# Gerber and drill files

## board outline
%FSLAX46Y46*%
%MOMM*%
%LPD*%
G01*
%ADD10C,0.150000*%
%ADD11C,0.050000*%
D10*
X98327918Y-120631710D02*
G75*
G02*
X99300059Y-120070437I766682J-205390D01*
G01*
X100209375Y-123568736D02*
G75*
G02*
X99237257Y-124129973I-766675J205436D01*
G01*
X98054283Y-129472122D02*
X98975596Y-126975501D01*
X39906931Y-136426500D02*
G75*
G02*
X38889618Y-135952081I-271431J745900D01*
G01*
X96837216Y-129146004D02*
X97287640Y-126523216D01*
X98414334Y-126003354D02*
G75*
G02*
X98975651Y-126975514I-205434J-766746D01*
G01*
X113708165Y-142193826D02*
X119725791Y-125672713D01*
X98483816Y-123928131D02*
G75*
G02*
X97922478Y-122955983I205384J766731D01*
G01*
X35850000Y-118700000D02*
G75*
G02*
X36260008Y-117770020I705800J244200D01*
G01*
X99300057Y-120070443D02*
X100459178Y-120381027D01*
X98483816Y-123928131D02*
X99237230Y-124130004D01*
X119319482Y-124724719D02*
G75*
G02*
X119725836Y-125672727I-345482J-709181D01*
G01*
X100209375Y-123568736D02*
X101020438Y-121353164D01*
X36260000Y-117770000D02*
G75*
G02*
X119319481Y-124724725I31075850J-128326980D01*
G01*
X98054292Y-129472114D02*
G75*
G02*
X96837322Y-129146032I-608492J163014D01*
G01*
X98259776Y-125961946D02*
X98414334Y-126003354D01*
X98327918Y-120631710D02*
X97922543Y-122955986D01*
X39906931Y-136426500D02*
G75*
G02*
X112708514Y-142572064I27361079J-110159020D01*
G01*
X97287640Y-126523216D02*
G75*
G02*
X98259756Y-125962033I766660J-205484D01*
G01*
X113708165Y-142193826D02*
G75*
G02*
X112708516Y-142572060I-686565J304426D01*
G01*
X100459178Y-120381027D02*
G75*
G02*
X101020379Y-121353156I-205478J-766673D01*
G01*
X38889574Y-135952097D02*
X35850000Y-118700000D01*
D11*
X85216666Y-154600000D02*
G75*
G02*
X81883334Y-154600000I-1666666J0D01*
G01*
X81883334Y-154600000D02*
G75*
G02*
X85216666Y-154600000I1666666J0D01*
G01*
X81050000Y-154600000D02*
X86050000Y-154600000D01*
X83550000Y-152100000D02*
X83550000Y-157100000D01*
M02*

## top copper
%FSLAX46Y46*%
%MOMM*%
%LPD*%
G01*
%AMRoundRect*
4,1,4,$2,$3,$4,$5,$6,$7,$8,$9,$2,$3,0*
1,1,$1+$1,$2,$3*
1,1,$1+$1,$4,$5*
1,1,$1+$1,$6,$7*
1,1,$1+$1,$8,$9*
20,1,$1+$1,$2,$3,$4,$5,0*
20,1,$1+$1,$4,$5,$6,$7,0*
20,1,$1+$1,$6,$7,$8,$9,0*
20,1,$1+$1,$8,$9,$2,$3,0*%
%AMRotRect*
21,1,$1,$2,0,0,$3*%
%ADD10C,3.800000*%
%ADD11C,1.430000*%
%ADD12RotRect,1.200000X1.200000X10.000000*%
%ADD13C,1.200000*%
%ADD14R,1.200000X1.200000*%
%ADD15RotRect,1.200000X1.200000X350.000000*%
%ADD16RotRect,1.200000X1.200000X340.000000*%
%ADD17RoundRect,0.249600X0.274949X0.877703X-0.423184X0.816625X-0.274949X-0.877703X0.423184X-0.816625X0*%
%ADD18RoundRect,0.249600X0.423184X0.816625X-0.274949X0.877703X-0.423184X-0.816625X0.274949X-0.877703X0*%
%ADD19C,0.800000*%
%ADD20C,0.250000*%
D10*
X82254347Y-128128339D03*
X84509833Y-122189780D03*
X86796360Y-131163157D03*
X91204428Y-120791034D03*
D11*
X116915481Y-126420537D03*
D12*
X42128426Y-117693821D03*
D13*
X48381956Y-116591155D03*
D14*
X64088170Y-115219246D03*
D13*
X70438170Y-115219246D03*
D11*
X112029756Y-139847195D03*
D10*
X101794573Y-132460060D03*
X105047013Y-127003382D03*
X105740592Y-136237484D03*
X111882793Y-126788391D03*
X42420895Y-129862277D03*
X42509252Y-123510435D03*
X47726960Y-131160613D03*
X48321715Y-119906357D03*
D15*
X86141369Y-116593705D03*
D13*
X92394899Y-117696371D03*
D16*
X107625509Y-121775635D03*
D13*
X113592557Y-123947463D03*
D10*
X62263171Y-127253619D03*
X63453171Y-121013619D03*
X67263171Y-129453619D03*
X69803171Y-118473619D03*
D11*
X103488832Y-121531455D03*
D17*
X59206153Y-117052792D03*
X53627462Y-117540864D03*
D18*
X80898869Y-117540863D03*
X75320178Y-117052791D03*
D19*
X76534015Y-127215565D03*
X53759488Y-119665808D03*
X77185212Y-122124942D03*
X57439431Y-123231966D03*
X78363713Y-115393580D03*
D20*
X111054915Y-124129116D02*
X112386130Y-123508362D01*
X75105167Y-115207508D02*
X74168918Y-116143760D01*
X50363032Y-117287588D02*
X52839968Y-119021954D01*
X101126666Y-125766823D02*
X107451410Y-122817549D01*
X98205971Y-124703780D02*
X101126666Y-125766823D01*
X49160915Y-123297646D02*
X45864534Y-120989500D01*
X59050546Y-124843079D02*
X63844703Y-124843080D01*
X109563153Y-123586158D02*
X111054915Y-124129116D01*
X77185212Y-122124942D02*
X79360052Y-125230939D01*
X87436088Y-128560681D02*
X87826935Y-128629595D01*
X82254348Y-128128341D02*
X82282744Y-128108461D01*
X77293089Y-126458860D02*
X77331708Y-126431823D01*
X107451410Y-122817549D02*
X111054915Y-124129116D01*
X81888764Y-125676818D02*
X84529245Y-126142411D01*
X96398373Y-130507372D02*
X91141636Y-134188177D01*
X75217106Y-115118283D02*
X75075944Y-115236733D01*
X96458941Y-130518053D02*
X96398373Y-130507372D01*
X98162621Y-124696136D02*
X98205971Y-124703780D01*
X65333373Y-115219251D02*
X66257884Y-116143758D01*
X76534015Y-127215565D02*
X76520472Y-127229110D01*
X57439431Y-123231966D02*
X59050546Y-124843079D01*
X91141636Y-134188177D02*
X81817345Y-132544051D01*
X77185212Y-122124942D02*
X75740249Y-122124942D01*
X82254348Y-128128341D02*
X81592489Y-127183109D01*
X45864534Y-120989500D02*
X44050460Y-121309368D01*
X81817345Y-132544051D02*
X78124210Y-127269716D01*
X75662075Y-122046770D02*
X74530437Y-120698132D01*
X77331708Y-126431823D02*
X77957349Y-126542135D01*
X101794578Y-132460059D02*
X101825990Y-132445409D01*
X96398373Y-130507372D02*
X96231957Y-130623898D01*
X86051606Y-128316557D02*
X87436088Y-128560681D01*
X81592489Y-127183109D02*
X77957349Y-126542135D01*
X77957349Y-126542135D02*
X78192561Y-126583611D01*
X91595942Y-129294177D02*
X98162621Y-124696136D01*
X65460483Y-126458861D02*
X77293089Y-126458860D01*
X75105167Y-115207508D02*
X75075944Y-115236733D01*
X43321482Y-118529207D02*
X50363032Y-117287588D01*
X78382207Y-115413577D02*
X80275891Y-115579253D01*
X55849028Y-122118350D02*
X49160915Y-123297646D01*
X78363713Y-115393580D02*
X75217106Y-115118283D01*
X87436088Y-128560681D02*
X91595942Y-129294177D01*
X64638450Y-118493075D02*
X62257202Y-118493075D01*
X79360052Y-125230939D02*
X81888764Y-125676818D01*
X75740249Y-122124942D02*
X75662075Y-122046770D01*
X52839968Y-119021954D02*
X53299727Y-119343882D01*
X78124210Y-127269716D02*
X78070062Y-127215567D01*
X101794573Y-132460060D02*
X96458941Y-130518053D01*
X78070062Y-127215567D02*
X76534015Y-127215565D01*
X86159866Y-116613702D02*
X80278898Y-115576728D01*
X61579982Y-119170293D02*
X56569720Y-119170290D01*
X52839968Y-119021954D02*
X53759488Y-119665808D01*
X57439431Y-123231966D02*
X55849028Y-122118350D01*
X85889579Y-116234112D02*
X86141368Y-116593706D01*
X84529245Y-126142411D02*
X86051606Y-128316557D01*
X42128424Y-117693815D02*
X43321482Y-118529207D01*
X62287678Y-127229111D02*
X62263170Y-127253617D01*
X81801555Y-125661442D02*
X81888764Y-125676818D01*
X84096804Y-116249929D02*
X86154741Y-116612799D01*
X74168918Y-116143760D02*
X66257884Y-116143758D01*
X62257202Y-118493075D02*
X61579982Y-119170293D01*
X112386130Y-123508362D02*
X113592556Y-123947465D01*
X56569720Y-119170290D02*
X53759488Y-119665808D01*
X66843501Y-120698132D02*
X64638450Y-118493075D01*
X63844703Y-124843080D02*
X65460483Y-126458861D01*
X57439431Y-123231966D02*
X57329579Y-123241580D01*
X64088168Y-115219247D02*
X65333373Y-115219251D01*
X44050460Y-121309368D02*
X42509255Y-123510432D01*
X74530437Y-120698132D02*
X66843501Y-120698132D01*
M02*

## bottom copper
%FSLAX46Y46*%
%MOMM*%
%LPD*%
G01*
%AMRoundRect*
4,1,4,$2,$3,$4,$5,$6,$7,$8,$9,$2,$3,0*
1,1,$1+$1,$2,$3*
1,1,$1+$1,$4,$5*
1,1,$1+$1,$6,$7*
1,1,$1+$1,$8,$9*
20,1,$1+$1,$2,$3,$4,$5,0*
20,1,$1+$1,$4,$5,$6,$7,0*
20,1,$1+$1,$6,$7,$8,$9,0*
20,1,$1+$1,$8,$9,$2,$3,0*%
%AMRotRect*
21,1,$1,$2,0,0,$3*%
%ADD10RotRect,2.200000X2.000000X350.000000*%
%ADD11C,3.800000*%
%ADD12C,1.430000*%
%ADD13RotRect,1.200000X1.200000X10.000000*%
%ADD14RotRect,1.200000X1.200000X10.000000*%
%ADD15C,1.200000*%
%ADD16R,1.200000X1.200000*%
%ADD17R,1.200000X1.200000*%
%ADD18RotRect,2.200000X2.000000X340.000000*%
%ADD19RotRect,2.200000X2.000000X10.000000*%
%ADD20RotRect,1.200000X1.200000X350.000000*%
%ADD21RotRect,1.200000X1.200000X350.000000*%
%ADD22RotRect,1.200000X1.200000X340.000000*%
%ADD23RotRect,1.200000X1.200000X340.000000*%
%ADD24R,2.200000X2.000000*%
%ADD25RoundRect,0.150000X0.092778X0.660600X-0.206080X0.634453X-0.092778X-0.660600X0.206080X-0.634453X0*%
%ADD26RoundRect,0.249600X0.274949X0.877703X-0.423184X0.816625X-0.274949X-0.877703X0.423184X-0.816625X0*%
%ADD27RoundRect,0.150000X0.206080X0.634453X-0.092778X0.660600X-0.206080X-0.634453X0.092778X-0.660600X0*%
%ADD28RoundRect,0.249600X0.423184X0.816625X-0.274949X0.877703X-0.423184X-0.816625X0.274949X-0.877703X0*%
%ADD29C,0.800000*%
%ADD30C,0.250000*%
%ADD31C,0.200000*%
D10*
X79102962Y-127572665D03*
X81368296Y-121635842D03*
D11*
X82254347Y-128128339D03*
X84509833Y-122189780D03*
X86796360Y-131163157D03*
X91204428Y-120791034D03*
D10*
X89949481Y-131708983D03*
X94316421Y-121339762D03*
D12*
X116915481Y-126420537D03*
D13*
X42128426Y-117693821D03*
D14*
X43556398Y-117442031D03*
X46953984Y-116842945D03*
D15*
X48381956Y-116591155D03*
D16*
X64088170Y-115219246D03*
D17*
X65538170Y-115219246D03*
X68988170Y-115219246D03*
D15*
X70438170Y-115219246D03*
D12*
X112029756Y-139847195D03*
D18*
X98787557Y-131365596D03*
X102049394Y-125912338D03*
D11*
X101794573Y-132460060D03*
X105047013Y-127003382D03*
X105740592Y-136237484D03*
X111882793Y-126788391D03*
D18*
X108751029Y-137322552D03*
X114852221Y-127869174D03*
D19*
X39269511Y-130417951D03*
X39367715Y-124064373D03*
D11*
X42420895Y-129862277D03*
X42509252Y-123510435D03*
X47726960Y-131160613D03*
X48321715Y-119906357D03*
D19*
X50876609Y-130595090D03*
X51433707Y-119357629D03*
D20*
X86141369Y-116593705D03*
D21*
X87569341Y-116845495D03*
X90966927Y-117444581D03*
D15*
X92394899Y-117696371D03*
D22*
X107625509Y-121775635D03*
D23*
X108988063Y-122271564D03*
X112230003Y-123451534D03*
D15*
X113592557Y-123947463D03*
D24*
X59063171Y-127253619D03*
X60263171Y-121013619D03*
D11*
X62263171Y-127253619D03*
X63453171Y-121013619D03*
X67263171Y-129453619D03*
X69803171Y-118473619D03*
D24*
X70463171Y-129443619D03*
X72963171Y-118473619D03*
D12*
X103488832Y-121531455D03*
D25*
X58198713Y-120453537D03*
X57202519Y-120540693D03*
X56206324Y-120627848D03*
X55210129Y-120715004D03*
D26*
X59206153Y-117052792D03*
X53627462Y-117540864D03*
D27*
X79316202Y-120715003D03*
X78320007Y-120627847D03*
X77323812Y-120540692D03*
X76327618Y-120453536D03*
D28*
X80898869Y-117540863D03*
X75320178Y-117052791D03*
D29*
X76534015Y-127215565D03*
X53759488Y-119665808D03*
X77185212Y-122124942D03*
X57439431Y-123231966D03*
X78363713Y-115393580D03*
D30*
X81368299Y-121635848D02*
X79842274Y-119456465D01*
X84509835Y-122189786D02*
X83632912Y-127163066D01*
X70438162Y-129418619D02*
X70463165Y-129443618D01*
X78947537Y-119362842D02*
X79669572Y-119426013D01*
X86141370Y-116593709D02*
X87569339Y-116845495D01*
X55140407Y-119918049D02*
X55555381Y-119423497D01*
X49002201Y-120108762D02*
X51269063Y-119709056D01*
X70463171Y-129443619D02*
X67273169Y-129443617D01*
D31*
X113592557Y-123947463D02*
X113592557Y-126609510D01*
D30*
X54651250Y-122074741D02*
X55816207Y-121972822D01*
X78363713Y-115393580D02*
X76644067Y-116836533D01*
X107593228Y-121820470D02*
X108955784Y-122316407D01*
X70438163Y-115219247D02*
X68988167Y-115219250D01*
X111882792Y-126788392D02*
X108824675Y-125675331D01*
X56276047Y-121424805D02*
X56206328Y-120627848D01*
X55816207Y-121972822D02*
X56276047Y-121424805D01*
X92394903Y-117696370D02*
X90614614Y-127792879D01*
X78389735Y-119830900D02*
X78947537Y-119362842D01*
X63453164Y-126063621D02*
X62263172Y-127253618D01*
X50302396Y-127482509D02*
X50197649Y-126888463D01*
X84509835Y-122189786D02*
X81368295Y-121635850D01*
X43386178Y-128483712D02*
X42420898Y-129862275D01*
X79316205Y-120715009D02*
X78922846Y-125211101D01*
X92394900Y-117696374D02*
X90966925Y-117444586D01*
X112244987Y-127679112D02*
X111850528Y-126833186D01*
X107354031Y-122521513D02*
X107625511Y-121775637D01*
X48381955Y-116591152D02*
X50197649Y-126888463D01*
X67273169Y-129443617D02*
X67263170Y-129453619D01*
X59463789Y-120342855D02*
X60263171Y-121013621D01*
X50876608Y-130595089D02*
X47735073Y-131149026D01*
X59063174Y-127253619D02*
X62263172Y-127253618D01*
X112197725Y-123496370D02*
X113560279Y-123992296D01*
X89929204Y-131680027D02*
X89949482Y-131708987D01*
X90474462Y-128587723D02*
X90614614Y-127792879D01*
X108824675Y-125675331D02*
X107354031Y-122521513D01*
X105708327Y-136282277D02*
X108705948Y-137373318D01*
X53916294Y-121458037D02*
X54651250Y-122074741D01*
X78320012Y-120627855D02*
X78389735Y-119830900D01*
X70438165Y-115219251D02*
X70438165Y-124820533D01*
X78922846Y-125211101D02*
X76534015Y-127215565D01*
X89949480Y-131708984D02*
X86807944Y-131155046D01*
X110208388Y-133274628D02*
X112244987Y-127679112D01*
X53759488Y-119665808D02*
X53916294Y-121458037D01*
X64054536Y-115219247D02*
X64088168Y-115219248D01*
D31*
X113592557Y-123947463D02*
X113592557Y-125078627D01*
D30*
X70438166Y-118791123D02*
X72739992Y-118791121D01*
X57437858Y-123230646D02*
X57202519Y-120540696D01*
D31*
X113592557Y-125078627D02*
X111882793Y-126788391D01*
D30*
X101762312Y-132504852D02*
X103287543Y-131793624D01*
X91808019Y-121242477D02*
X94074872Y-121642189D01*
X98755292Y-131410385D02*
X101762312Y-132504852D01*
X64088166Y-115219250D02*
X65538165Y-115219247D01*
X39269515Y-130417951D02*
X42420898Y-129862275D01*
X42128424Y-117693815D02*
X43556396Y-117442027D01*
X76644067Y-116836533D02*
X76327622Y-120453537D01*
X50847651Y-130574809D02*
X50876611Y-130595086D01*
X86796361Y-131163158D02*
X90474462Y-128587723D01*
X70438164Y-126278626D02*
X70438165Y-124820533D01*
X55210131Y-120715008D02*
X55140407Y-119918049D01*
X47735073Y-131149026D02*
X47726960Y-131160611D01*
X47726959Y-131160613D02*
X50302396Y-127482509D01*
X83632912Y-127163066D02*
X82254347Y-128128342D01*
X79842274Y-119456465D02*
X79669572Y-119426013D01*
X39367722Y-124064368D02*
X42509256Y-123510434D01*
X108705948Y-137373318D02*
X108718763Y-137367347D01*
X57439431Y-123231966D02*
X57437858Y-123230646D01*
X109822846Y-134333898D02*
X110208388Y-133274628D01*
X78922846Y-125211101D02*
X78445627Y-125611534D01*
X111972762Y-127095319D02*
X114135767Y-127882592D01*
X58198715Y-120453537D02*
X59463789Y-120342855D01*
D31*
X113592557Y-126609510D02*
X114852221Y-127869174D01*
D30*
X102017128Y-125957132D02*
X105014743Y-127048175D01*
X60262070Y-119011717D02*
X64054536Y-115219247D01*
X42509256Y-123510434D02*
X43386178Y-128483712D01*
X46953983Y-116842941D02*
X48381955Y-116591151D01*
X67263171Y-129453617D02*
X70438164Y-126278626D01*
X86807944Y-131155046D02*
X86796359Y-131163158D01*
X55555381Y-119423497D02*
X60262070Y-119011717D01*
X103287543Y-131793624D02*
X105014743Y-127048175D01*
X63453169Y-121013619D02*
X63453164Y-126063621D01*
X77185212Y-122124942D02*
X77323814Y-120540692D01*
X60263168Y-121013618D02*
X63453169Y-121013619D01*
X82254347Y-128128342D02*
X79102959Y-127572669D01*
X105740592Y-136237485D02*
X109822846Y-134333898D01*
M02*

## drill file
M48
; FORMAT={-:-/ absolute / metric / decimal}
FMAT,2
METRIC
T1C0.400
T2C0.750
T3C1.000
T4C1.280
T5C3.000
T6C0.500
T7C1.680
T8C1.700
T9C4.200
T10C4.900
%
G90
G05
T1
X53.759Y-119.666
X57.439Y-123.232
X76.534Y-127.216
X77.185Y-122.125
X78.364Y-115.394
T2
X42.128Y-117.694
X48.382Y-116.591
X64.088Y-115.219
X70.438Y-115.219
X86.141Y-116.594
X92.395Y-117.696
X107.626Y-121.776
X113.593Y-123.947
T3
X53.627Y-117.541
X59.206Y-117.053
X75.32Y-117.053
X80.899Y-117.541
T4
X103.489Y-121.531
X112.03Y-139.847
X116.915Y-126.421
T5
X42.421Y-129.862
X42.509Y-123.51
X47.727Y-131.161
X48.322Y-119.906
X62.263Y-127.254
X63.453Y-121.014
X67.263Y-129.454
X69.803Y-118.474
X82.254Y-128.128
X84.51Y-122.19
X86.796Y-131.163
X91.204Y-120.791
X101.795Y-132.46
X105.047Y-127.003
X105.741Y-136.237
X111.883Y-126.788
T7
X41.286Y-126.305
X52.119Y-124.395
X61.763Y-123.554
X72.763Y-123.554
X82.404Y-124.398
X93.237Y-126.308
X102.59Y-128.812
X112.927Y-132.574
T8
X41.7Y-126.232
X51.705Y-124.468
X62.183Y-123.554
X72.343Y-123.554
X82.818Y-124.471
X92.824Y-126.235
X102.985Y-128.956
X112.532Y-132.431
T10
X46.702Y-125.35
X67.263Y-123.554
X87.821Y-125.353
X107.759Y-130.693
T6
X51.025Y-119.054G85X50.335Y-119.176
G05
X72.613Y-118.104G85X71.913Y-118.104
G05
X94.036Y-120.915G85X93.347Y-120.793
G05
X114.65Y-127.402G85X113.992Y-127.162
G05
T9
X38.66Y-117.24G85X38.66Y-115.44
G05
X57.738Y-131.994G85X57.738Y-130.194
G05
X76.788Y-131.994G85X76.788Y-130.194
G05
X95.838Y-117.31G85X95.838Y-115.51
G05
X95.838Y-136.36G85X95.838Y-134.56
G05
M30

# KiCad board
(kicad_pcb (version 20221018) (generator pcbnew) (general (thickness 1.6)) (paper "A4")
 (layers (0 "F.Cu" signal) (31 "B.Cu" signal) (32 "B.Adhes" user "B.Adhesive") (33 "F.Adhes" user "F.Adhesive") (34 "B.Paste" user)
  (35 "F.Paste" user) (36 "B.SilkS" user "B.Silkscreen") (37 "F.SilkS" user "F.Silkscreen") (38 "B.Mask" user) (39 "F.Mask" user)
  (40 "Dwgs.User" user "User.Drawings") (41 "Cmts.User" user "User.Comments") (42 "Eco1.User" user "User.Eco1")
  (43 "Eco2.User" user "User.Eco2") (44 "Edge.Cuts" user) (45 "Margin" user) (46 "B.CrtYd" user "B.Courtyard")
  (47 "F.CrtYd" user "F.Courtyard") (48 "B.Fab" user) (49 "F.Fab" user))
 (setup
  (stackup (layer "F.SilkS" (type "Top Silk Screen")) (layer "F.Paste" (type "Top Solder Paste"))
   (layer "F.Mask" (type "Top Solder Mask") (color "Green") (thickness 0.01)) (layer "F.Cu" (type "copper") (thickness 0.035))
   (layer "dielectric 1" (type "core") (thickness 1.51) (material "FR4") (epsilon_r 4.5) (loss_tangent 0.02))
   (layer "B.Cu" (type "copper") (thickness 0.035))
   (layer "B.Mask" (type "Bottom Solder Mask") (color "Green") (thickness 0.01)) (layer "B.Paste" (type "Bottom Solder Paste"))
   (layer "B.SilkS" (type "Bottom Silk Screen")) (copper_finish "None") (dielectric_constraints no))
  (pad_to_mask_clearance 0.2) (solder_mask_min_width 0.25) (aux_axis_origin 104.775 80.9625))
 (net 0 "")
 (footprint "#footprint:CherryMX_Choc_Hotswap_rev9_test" (layer "F.Cu") (at 87.820884 125.352791 -10)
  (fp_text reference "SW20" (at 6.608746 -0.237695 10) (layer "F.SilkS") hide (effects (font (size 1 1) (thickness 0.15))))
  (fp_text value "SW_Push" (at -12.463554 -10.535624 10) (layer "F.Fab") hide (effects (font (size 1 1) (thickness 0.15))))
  (pad "" np_thru_hole circle (at -5.5 0 80) (size 1.68 1.68) (drill 1.68) (layers "F&B.Cu" "*.Mask"))
  (pad "" np_thru_hole circle (at -5.08 0 350) (size 1.7 1.7) (drill 1.7) (layers "*.Cu" "*.Mask"))
  (pad "" np_thru_hole circle (at 0 0 80) (size 4.9 4.9) (drill 4.9) (layers "F&B.Cu" "*.Mask"))
  (pad "" np_thru_hole oval (at 5 -5.45 170) (size 1.2 0.5) (drill oval 1.2 0.5) (layers "F&B.Cu" "*.Mask"))
  (pad "" np_thru_hole circle (at 5.08 0 350) (size 1.7 1.7) (drill 1.7) (layers "*.Cu" "*.Mask"))
  (pad "" np_thru_hole circle (at 5.5 0 80) (size 1.68 1.68) (drill 1.68) (layers "F&B.Cu" "*.Mask"))
  (pad "1" smd rect (at -8.2 3.7 350) (size 2.2 2) (layers "B.Cu" "B.Paste" "B.Mask"))
  (pad "1" smd rect (at -7 -2.54 350) (size 2.2 2) (layers "B.Cu" "B.Paste" "B.Mask"))
  (pad "1" thru_hole circle (at -5 3.7 80) (size 3.8 3.8) (drill 3) (layers "*.Cu" "B.Mask"))
  (pad "1" thru_hole circle (at -3.81 -2.54 170) (size 3.8 3.8) (drill 3) (layers "*.Cu" "B.Mask"))
  (pad "2" thru_hole circle (at 0 5.9 80) (size 3.8 3.8) (drill 3) (layers "*.Cu" "B.Mask"))
  (pad "2" thru_hole circle (at 2.54 -5.08 170) (size 3.8 3.8) (drill 3) (layers "*.Cu" "B.Mask"))
  (pad "2" smd rect (at 3.2 5.89 350) (size 2.2 2) (layers "B.Cu" "B.Paste" "B.Mask"))
  (pad "2" smd rect (at 5.7 -5.08 350) (size 2.2 2) (layers "B.Cu" "B.Paste" "B.Mask")))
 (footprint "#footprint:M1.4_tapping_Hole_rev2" (layer "F.Cu") (at 116.915481 126.420537)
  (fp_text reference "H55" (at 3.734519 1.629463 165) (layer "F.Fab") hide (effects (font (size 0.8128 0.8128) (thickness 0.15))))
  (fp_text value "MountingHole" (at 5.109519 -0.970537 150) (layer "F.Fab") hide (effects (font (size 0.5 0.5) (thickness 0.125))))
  (pad "" thru_hole circle (at 0 0) (size 1.43 1.43) (drill 1.28) (layers "*.Cu" "*.Mask")))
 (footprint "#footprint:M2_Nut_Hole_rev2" (layer "F.Cu") (at 76.788168 131.09425 90)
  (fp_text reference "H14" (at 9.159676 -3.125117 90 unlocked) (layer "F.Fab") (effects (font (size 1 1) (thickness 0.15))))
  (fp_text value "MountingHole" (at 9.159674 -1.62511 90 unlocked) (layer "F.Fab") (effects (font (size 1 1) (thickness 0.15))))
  (pad "" np_thru_hole oval (at 0 0 90) (size 6 4.2) (drill oval 6 4.2) (layers "F&B.Cu" "*.Mask")))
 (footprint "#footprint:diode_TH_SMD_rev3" (layer "F.Cu") (at 45.255191 117.142488 10)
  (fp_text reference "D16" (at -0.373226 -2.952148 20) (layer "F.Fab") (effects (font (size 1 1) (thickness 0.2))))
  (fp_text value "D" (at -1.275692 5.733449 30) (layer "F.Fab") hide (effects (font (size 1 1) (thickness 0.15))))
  (pad "1" thru_hole rect (at -3.175 0 10) (size 1.2 1.2) (drill 0.75) (layers "*.Cu" "B.Mask"))
  (pad "1" smd rect (at -1.725 0 10) (size 1.2 1.2) (layers "B.Cu" "B.Paste" "B.Mask"))
  (pad "2" smd rect (at 1.725 0 10) (size 1.2 1.2) (layers "B.Cu" "B.Paste" "B.Mask"))
  (pad "2" thru_hole circle (at 3.175 0 10) (size 1.2 1.2) (drill 0.75) (layers "*.Cu" "B.Mask")))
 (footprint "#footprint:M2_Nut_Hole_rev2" (layer "F.Cu") (at 38.688172 116.409876 90)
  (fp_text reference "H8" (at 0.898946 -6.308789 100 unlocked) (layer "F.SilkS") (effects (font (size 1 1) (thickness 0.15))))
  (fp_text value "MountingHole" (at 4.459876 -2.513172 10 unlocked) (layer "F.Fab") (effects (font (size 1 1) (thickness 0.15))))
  (pad "" np_thru_hole oval (at 0.069876 -0.028172 90) (size 6 4.2) (drill oval 6 4.2) (layers "F&B.Cu" "*.Mask")))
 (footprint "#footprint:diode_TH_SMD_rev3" (layer "F.Cu") (at 67.26317 115.219246)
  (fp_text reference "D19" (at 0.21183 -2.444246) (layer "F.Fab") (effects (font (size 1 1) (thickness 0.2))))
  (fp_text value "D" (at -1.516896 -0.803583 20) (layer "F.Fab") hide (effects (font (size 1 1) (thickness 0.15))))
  (pad "1" thru_hole rect (at -3.175 0) (size 1.2 1.2) (drill 0.75) (layers "*.Cu" "B.Mask"))
  (pad "1" smd rect (at -1.725 0) (size 1.2 1.2) (layers "B.Cu" "B.Paste" "B.Mask"))
  (pad "2" smd rect (at 1.725 0) (size 1.2 1.2) (layers "B.Cu" "B.Paste" "B.Mask"))
  (pad "2" thru_hole circle (at 3.175 0) (size 1.2 1.2) (drill 0.75) (layers "*.Cu" "B.Mask")))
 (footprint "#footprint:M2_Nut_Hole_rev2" (layer "F.Cu") (at 95.838173 135.459873 90)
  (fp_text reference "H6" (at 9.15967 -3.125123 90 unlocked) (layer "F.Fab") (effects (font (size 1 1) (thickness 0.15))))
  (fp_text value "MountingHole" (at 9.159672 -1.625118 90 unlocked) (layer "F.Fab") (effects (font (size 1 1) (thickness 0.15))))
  (pad "" np_thru_hole oval (at 0 0 90) (size 6 4.2) (drill oval 6 4.2) (layers "F&B.Cu" "*.Mask")))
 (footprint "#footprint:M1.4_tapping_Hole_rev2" (layer "F.Cu") (at 31.044945 121.53341)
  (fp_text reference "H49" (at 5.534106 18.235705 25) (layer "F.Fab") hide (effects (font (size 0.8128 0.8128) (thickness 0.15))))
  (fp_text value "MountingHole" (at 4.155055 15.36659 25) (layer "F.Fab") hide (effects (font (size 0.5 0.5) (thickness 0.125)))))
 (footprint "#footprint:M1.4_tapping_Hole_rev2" (layer "F.Cu") (at 112.029756 139.847195)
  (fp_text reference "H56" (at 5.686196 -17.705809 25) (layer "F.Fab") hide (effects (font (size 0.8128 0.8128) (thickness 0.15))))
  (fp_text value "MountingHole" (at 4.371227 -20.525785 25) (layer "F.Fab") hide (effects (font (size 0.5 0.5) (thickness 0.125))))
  (pad "" thru_hole circle (at 0 0) (size 1.43 1.43) (drill 1.28) (layers "*.Cu" "*.Mask")))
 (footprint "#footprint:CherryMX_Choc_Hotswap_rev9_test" (layer "F.Cu") (at 107.758511 130.693298 -20)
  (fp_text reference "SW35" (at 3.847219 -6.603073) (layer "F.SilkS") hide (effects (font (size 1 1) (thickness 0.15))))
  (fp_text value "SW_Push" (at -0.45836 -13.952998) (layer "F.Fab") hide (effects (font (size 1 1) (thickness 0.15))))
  (pad "" np_thru_hole circle (at -5.5 0 70) (size 1.68 1.68) (drill 1.68) (layers "F&B.Cu" "*.Mask"))
  (pad "" np_thru_hole circle (at -5.08 0 340) (size 1.7 1.7) (drill 1.7) (layers "*.Cu" "*.Mask"))
  (pad "" np_thru_hole circle (at 0 0 70) (size 4.9 4.9) (drill 4.9) (layers "F&B.Cu" "*.Mask"))
  (pad "" np_thru_hole oval (at 5 -5.45 160) (size 1.2 0.5) (drill oval 1.2 0.5) (layers "F&B.Cu" "*.Mask"))
  (pad "" np_thru_hole circle (at 5.08 0 340) (size 1.7 1.7) (drill 1.7) (layers "*.Cu" "*.Mask"))
  (pad "" np_thru_hole circle (at 5.5 0 70) (size 1.68 1.68) (drill 1.68) (layers "F&B.Cu" "*.Mask"))
  (pad "1" smd rect (at -8.2 3.7 340) (size 2.2 2) (layers "B.Cu" "B.Paste" "B.Mask"))
  (pad "1" smd rect (at -7 -2.54 340) (size 2.2 2) (layers "B.Cu" "B.Paste" "B.Mask"))
  (pad "1" thru_hole circle (at -5 3.7 70) (size 3.8 3.8) (drill 3) (layers "*.Cu" "B.Mask"))
  (pad "1" thru_hole circle (at -3.81 -2.54 160) (size 3.8 3.8) (drill 3) (layers "*.Cu" "B.Mask"))
  (pad "2" thru_hole circle (at 0 5.9 70) (size 3.8 3.8) (drill 3) (layers "*.Cu" "B.Mask"))
  (pad "2" thru_hole circle (at 2.54 -5.08 160) (size 3.8 3.8) (drill 3) (layers "*.Cu" "B.Mask"))
  (pad "2" smd rect (at 3.2 5.89 340) (size 2.2 2) (layers "B.Cu" "B.Paste" "B.Mask"))
  (pad "2" smd rect (at 5.7 -5.08 340) (size 2.2 2) (layers "B.Cu" "B.Paste" "B.Mask")))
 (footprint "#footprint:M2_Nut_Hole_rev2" (layer "F.Cu") (at 95.83817 116.409867 90)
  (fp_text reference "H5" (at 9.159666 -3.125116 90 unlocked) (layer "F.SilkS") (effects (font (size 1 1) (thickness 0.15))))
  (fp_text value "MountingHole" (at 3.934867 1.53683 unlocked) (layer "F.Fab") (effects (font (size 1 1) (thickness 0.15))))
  (pad "" np_thru_hole oval (at 0 0 90) (size 6 4.2) (drill oval 6 4.2) (layers "F&B.Cu" "*.Mask")))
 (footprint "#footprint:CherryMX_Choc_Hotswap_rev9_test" (layer "F.Cu") (at 46.702436 125.350247 10)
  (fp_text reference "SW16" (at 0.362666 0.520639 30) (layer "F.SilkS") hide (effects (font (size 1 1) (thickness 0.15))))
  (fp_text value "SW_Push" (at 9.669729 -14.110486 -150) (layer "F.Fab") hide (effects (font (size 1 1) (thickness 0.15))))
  (pad "" np_thru_hole circle (at -5.5 0 100) (size 1.68 1.68) (drill 1.68) (layers "F&B.Cu" "*.Mask"))
  (pad "" np_thru_hole circle (at -5.08 0 10) (size 1.7 1.7) (drill 1.7) (layers "*.Cu" "*.Mask"))
  (pad "" np_thru_hole circle (at 0 0 100) (size 4.9 4.9) (drill 4.9) (layers "F&B.Cu" "*.Mask"))
  (pad "" np_thru_hole oval (at 5 -5.45 190) (size 1.2 0.5) (drill oval 1.2 0.5) (layers "F&B.Cu" "*.Mask"))
  (pad "" np_thru_hole circle (at 5.08 0 10) (size 1.7 1.7) (drill 1.7) (layers "*.Cu" "*.Mask"))
  (pad "" np_thru_hole circle (at 5.5 0 100) (size 1.68 1.68) (drill 1.68) (layers "F&B.Cu" "*.Mask"))
  (pad "1" smd rect (at -8.2 3.7 10) (size 2.2 2) (layers "B.Cu" "B.Paste" "B.Mask"))
  (pad "1" smd rect (at -7 -2.54 10) (size 2.2 2) (layers "B.Cu" "B.Paste" "B.Mask"))
  (pad "1" thru_hole circle (at -5 3.7 100) (size 3.8 3.8) (drill 3) (layers "*.Cu" "B.Mask"))
  (pad "1" thru_hole circle (at -3.81 -2.54 190) (size 3.8 3.8) (drill 3) (layers "*.Cu" "B.Mask"))
  (pad "2" thru_hole circle (at 0 5.9 100) (size 3.8 3.8) (drill 3) (layers "*.Cu" "B.Mask"))
  (pad "2" thru_hole circle (at 2.54 -5.08 190) (size 3.8 3.8) (drill 3) (layers "*.Cu" "B.Mask"))
  (pad "2" smd rect (at 3.2 5.89 10) (size 2.2 2) (layers "B.Cu" "B.Paste" "B.Mask"))
  (pad "2" smd rect (at 5.7 -5.08 10) (size 2.2 2) (layers "B.Cu" "B.Paste" "B.Mask")))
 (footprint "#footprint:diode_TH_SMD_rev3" (layer "F.Cu") (at 89.268134 117.145038 -10)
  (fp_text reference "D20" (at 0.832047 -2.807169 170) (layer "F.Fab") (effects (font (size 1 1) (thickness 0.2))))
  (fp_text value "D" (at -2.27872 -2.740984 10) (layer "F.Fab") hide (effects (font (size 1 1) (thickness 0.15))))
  (pad "1" thru_hole rect (at -3.175 0 350) (size 1.2 1.2) (drill 0.75) (layers "*.Cu" "B.Mask"))
  (pad "1" smd rect (at -1.725 0 350) (size 1.2 1.2) (layers "B.Cu" "B.Paste" "B.Mask"))
  (pad "2" smd rect (at 1.725 0 350) (size 1.2 1.2) (layers "B.Cu" "B.Paste" "B.Mask"))
  (pad "2" thru_hole circle (at 3.175 0 350) (size 1.2 1.2) (drill 0.75) (layers "*.Cu" "B.Mask")))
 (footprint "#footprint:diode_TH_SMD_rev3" (layer "F.Cu") (at 110.609033 122.861549 -20)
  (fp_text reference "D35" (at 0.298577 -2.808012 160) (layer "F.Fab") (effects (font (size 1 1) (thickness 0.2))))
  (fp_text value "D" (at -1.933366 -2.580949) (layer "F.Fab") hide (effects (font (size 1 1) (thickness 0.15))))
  (pad "1" thru_hole rect (at -3.175 0 340) (size 1.2 1.2) (drill 0.75) (layers "*.Cu" "B.Mask"))
  (pad "1" smd rect (at -1.725 0 340) (size 1.2 1.2) (layers "B.Cu" "B.Paste" "B.Mask"))
  (pad "2" smd rect (at 1.725 0 340) (size 1.2 1.2) (layers "B.Cu" "B.Paste" "B.Mask"))
  (pad "2" thru_hole circle (at 3.175 0 340) (size 1.2 1.2) (drill 0.75) (layers "*.Cu" "B.Mask")))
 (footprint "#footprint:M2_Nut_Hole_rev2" (layer "F.Cu") (at 57.738174 131.094247 90)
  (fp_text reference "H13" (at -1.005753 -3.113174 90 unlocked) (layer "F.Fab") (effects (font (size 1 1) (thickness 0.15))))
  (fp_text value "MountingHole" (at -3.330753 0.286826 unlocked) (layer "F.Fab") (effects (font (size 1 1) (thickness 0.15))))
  (pad "" np_thru_hole oval (at 0 0 90) (size 6 4.2) (drill oval 6 4.2) (layers "F&B.Cu" "*.Mask")))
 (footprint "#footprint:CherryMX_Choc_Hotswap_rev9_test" (layer "F.Cu") (at 67.263171 123.553619)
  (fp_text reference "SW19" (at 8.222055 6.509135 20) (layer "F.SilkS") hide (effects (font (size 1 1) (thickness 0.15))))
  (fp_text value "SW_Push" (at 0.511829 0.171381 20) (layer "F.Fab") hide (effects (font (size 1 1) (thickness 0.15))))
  (pad "" np_thru_hole circle (at -5.5 0 90) (size 1.68 1.68) (drill 1.68) (layers "F&B.Cu" "*.Mask"))
  (pad "" np_thru_hole circle (at -5.08 0) (size 1.7 1.7) (drill 1.7) (layers "*.Cu" "*.Mask"))
  (pad "" np_thru_hole circle (at 0 0 90) (size 4.9 4.9) (drill 4.9) (layers "F&B.Cu" "*.Mask"))
  (pad "" np_thru_hole oval (at 5 -5.45 180) (size 1.2 0.5) (drill oval 1.2 0.5) (layers "F&B.Cu" "*.Mask"))
  (pad "" np_thru_hole circle (at 5.08 0) (size 1.7 1.7) (drill 1.7) (layers "*.Cu" "*.Mask"))
  (pad "" np_thru_hole circle (at 5.5 0 90) (size 1.68 1.68) (drill 1.68) (layers "F&B.Cu" "*.Mask"))
  (pad "1" smd rect (at -8.2 3.7) (size 2.2 2) (layers "B.Cu" "B.Paste" "B.Mask"))
  (pad "1" smd rect (at -7 -2.54) (size 2.2 2) (layers "B.Cu" "B.Paste" "B.Mask"))
  (pad "1" thru_hole circle (at -5 3.7 90) (size 3.8 3.8) (drill 3) (layers "*.Cu" "B.Mask"))
  (pad "1" thru_hole circle (at -3.81 -2.54 180) (size 3.8 3.8) (drill 3) (layers "*.Cu" "B.Mask"))
  (pad "2" thru_hole circle (at 0 5.9 90) (size 3.8 3.8) (drill 3) (layers "*.Cu" "B.Mask"))
  (pad "2" thru_hole circle (at 2.54 -5.08 180) (size 3.8 3.8) (drill 3) (layers "*.Cu" "B.Mask"))
  (pad "2" smd rect (at 3.2 5.89) (size 2.2 2) (layers "B.Cu" "B.Paste" "B.Mask"))
  (pad "2" smd rect (at 5.7 -5.08) (size 2.2 2) (layers "B.Cu" "B.Paste" "B.Mask")))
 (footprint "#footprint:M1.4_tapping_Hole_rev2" (layer "F.Cu") (at 17.628748 126.416282)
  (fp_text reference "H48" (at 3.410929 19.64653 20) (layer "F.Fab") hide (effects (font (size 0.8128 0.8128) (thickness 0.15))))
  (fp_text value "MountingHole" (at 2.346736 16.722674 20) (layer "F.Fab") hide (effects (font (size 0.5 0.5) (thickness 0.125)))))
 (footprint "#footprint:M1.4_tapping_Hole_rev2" (layer "F.Cu") (at 103.488832 121.531455)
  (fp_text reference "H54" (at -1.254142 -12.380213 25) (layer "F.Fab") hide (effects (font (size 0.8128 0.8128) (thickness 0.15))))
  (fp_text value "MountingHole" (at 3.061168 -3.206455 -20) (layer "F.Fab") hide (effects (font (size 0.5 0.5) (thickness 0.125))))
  (pad "" thru_hole circle (at 0 0) (size 1.43 1.43) (drill 1.28) (layers "*.Cu" "*.Mask")))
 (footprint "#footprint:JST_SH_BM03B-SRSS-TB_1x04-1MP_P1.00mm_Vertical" (layer "B.Cu") (at 56.547541 118.79112 -175)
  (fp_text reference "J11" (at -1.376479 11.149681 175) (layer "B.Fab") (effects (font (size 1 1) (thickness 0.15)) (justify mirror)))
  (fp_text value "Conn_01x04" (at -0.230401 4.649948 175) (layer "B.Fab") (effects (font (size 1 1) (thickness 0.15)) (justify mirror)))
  (pad "1" smd roundrect (at -1.5 -1.8 185) (size 0.6 1.6) (layers "B.Cu" "B.Paste" "B.Mask") (roundrect_rratio 0.25))
  (pad "2" smd roundrect (at -0.5 -1.8 185) (size 0.6 1.6) (layers "B.Cu" "B.Paste" "B.Mask") (roundrect_rratio 0.25))
  (pad "3" smd roundrect (at 0.5 -1.8 185) (size 0.6 1.6) (layers "B.Cu" "B.Paste" "B.Mask") (roundrect_rratio 0.25))
  (pad "4" smd roundrect (at 1.5 -1.8 185) (size 0.6 1.6) (layers "B.Cu" "B.Paste" "B.Mask") (roundrect_rratio 0.25))
  (pad "MP" thru_hole roundrect (at -2.8 1.5 185) (size 1.2 2.2) (drill 1) (layers "*.Cu" "*.Mask") (roundrect_rratio 0.208))
  (pad "MP" thru_hole roundrect (at 2.8 1.5 185) (size 1.2 2.2) (drill 1) (layers "*.Cu" "*.Mask") (roundrect_rratio 0.208)))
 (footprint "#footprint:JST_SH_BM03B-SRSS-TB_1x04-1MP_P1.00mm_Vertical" (layer "B.Cu") (at 77.97879 118.791119 175)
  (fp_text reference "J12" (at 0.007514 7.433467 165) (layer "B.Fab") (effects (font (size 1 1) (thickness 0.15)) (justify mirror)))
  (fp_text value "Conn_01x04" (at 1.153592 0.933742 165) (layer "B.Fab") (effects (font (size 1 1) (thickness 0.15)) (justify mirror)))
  (pad "1" smd roundrect (at -1.5 -1.8 175) (size 0.6 1.6) (layers "B.Cu" "B.Paste" "B.Mask") (roundrect_rratio 0.25))
  (pad "2" smd roundrect (at -0.5 -1.8 175) (size 0.6 1.6) (layers "B.Cu" "B.Paste" "B.Mask") (roundrect_rratio 0.25))
  (pad "3" smd roundrect (at 0.5 -1.8 175) (size 0.6 1.6) (layers "B.Cu" "B.Paste" "B.Mask") (roundrect_rratio 0.25))
  (pad "4" smd roundrect (at 1.5 -1.8 175) (size 0.6 1.6) (layers "B.Cu" "B.Paste" "B.Mask") (roundrect_rratio 0.25))
  (pad "MP" thru_hole roundrect (at -2.8 1.5 175) (size 1.2 2.2) (drill 1) (layers "*.Cu" "*.Mask") (roundrect_rratio 0.208))
  (pad "MP" thru_hole roundrect (at 2.8 1.5 175) (size 1.2 2.2) (drill 1) (layers "*.Cu" "*.Mask") (roundrect_rratio 0.208)))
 (gr_arc (start 98.327918 120.63171) (mid 98.697746 120.149741) (end 99.300057 120.070445) (stroke (width 0.15) (type solid))
  (layer "Edge.Cuts"))
 (gr_arc (start 100.209375 123.568736) (mid 99.839555 124.050709) (end 99.237246 124.130013) (stroke (width 0.15) (type solid))
  (layer "Edge.Cuts"))
 (gr_line (start 98.054283 129.472122) (end 98.975596 126.975501) (stroke (width 0.15) (type solid)) (layer "Edge.Cuts"))
 (gr_arc (start 39.906931 136.4265) (mid 39.3 136.4) (end 38.889574 135.952097) (stroke (width 0.15) (type solid)) (layer "Edge.Cuts"))
 (gr_line (start 96.837216 129.146004) (end 97.28764 126.523216) (stroke (width 0.15) (type solid)) (layer "Edge.Cuts"))
 (gr_arc (start 98.414334 126.003354) (mid 98.896307 126.373185) (end 98.975603 126.975501) (stroke (width 0.15) (type solid))
  (layer "Edge.Cuts"))
 (gr_line (start 113.708165 142.193826) (end 119.725791 125.672713) (stroke (width 0.15) (type solid)) (layer "Edge.Cuts"))
 (gr_arc (start 98.483816 123.928131) (mid 98.001842 123.558309) (end 97.922538 122.955999) (stroke (width 0.15) (type solid))
  (layer "Edge.Cuts"))
 (gr_arc (start 35.85 118.7) (mid 35.872407 118.154502) (end 36.26 117.77) (stroke (width 0.15) (type solid)) (layer "Edge.Cuts"))
 (gr_line (start 99.300057 120.070443) (end 100.459178 120.381027) (stroke (width 0.15) (type solid)) (layer "Edge.Cuts"))
 (gr_line (start 98.483816 123.928131) (end 99.23723 124.130004) (stroke (width 0.15) (type solid)) (layer "Edge.Cuts"))
 (gr_arc (start 119.319482 124.724719) (mid 119.699035 125.123112) (end 119.725791 125.672713) (stroke (width 0.15) (type solid))
  (layer "Edge.Cuts"))
 (gr_line (start 100.209375 123.568736) (end 101.020438 121.353164) (stroke (width 0.15) (type solid)) (layer "Edge.Cuts"))
 (gr_arc (start 36.26 117.77) (mid 78.352542 114.521317) (end 119.319482 124.724722) (stroke (width 0.15) (type solid)) (layer "Edge.Cuts"))
 (gr_arc (start 98.054292 129.472114) (mid 97.282699 129.917597) (end 96.837216 129.146004) (stroke (width 0.15) (type solid))
  (layer "Edge.Cuts"))
 (gr_line (start 98.259776 125.961946) (end 98.414334 126.003354) (stroke (width 0.15) (type solid)) (layer "Edge.Cuts"))
 (gr_line (start 98.327918 120.63171) (end 97.922543 122.955986) (stroke (width 0.15) (type solid)) (layer "Edge.Cuts"))
 (gr_arc (start 39.906931 136.4265) (mid 76.8157 133.481675) (end 112.708513 142.572066) (stroke (width 0.15) (type solid))
  (layer "Edge.Cuts"))
 (gr_arc (start 97.28764 126.523216) (mid 97.657467 126.041245) (end 98.259779 125.961947) (stroke (width 0.15) (type solid))
  (layer "Edge.Cuts"))
 (gr_arc (start 113.708165 142.193826) (mid 113.287377 142.591836) (end 112.708512 142.572069) (stroke (width 0.15) (type solid))
  (layer "Edge.Cuts"))
 (gr_arc (start 100.459178 120.381027) (mid 100.941146 120.750859) (end 101.020439 121.353172) (stroke (width 0.15) (type solid))
  (layer "Edge.Cuts"))
 (gr_line (start 38.889574 135.952097) (end 35.85 118.7) (stroke (width 0.15) (type solid)) (layer "Edge.Cuts"))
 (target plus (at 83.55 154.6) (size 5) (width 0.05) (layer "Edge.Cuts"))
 (segment (start 111.054915 124.129116) (end 112.38613 123.508362) (width 0.25) (layer "F.Cu") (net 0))
 (segment (start 75.105167 115.207508) (end 74.168918 116.14376) (width 0.25) (layer "F.Cu") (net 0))
 (segment (start 50.363032 117.287588) (end 52.839968 119.021954) (width 0.25) (layer "F.Cu") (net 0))
 (segment (start 101.126666 125.766823) (end 107.45141 122.817549) (width 0.25) (layer "F.Cu") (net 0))
 (segment (start 98.205971 124.70378) (end 101.126666 125.766823) (width 0.25) (layer "F.Cu") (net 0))
 (segment (start 49.160915 123.297646) (end 45.864534 120.9895) (width 0.25) (layer "F.Cu") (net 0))
 (segment (start 59.050546 124.843079) (end 63.844703 124.84308) (width 0.25) (layer "F.Cu") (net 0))
 (segment (start 109.563153 123.586158) (end 111.054915 124.129116) (width 0.25) (layer "F.Cu") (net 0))
 (segment (start 77.185212 122.124942) (end 79.360052 125.230939) (width 0.25) (layer "F.Cu") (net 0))
 (segment (start 87.436088 128.560681) (end 87.826935 128.629595) (width 0.25) (layer "F.Cu") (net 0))
 (segment (start 82.254348 128.128341) (end 82.282744 128.108461) (width 0.25) (layer "F.Cu") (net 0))
 (segment (start 77.293089 126.45886) (end 77.331708 126.431823) (width 0.25) (layer "F.Cu") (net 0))
 (segment (start 107.45141 122.817549) (end 111.054915 124.129116) (width 0.25) (layer "F.Cu") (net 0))
 (segment (start 81.888764 125.676818) (end 84.529245 126.142411) (width 0.25) (layer "F.Cu") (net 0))
 (segment (start 96.398373 130.507372) (end 91.141636 134.188177) (width 0.25) (layer "F.Cu") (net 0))
 (segment (start 75.217106 115.118283) (end 75.075944 115.236733) (width 0.25) (layer "F.Cu") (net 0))
 (segment (start 96.458941 130.518053) (end 96.398373 130.507372) (width 0.25) (layer "F.Cu") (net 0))
 (segment (start 98.162621 124.696136) (end 98.205971 124.70378) (width 0.25) (layer "F.Cu") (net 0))
 (segment (start 65.333373 115.219251) (end 66.257884 116.143758) (width 0.25) (layer "F.Cu") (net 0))
 (segment (start 76.534015 127.215565) (end 76.520472 127.22911) (width 0.25) (layer "F.Cu") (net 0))
 (segment (start 57.439431 123.231966) (end 59.050546 124.843079) (width 0.25) (layer "F.Cu") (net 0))
 (segment (start 91.141636 134.188177) (end 81.817345 132.544051) (width 0.25) (layer "F.Cu") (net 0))
 (segment (start 77.185212 122.124942) (end 75.740249 122.124942) (width 0.25) (layer "F.Cu") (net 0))
 (segment (start 82.254348 128.128341) (end 81.592489 127.183109) (width 0.25) (layer "F.Cu") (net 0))
 (segment (start 45.864534 120.9895) (end 44.05046 121.309368) (width 0.25) (layer "F.Cu") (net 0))
 (segment (start 81.817345 132.544051) (end 78.12421 127.269716) (width 0.25) (layer "F.Cu") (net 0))
 (segment (start 75.662075 122.04677) (end 74.530437 120.698132) (width 0.25) (layer "F.Cu") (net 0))
 (segment (start 77.331708 126.431823) (end 77.957349 126.542135) (width 0.25) (layer "F.Cu") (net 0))
 (segment (start 101.794578 132.460059) (end 101.82599 132.445409) (width 0.25) (layer "F.Cu") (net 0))
 (segment (start 96.398373 130.507372) (end 96.231957 130.623898) (width 0.25) (layer "F.Cu") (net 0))
 (segment (start 86.051606 128.316557) (end 87.436088 128.560681) (width 0.25) (layer "F.Cu") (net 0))
 (segment (start 81.592489 127.183109) (end 77.957349 126.542135) (width 0.25) (layer "F.Cu") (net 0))
 (segment (start 77.957349 126.542135) (end 78.192561 126.583611) (width 0.25) (layer "F.Cu") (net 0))
 (segment (start 91.595942 129.294177) (end 98.162621 124.696136) (width 0.25) (layer "F.Cu") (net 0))
 (segment (start 65.460483 126.458861) (end 77.293089 126.45886) (width 0.25) (layer "F.Cu") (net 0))
 (segment (start 75.105167 115.207508) (end 75.075944 115.236733) (width 0.25) (layer "F.Cu") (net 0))
 (segment (start 43.321482 118.529207) (end 50.363032 117.287588) (width 0.25) (layer "F.Cu") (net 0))
 (segment (start 78.382207 115.413577) (end 80.275891 115.579253) (width 0.25) (layer "F.Cu") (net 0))
 (segment (start 55.849028 122.11835) (end 49.160915 123.297646) (width 0.25) (layer "F.Cu") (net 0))
 (segment (start 78.363713 115.39358) (end 75.217106 115.118283) (width 0.25) (layer "F.Cu") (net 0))
 (segment (start 87.436088 128.560681) (end 91.595942 129.294177) (width 0.25) (layer "F.Cu") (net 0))
 (segment (start 64.63845 118.493075) (end 62.257202 118.493075) (width 0.25) (layer "F.Cu") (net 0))
 (segment (start 79.360052 125.230939) (end 81.888764 125.676818) (width 0.25) (layer "F.Cu") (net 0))
 (segment (start 75.740249 122.124942) (end 75.662075 122.04677) (width 0.25) (layer "F.Cu") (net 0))
 (segment (start 52.839968 119.021954) (end 53.299727 119.343882) (width 0.25) (layer "F.Cu") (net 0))
 (segment (start 78.12421 127.269716) (end 78.070062 127.215567) (width 0.25) (layer "F.Cu") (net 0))
 (segment (start 101.794573 132.46006) (end 96.458941 130.518053) (width 0.25) (layer "F.Cu") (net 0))
 (segment (start 78.070062 127.215567) (end 76.534015 127.215565) (width 0.25) (layer "F.Cu") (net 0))
 (segment (start 86.159866 116.613702) (end 80.278898 115.576728) (width 0.25) (layer "F.Cu") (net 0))
 (segment (start 61.579982 119.170293) (end 56.56972 119.17029) (width 0.25) (layer "F.Cu") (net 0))
 (segment (start 52.839968 119.021954) (end 53.759488 119.665808) (width 0.25) (layer "F.Cu") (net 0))
 (segment (start 57.439431 123.231966) (end 55.849028 122.11835) (width 0.25) (layer "F.Cu") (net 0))
 (segment (start 85.889579 116.234112) (end 86.141368 116.593706) (width 0.25) (layer "F.Cu") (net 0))
 (segment (start 84.529245 126.142411) (end 86.051606 128.316557) (width 0.25) (layer "F.Cu") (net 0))
 (segment (start 42.128424 117.693815) (end 43.321482 118.529207) (width 0.25) (layer "F.Cu") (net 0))
 (segment (start 62.287678 127.229111) (end 62.26317 127.253617) (width 0.25) (layer "F.Cu") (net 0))
 (segment (start 81.801555 125.661442) (end 81.888764 125.676818) (width 0.25) (layer "F.Cu") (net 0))
 (segment (start 84.096804 116.249929) (end 86.154741 116.612799) (width 0.25) (layer "F.Cu") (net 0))
 (segment (start 74.168918 116.14376) (end 66.257884 116.143758) (width 0.25) (layer "F.Cu") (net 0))
 (segment (start 62.257202 118.493075) (end 61.579982 119.170293) (width 0.25) (layer "F.Cu") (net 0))
 (segment (start 112.38613 123.508362) (end 113.592556 123.947465) (width 0.25) (layer "F.Cu") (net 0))
 (segment (start 56.56972 119.17029) (end 53.759488 119.665808) (width 0.25) (layer "F.Cu") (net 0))
 (segment (start 66.843501 120.698132) (end 64.63845 118.493075) (width 0.25) (layer "F.Cu") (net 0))
 (segment (start 63.844703 124.84308) (end 65.460483 126.458861) (width 0.25) (layer "F.Cu") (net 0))
 (segment (start 57.439431 123.231966) (end 57.329579 123.24158) (width 0.25) (layer "F.Cu") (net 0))
 (segment (start 64.088168 115.219247) (end 65.333373 115.219251) (width 0.25) (layer "F.Cu") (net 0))
 (segment (start 44.05046 121.309368) (end 42.509255 123.510432) (width 0.25) (layer "F.Cu") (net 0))
 (segment (start 74.530437 120.698132) (end 66.843501 120.698132) (width 0.25) (layer "F.Cu") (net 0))
 (via (at 76.534015 127.215565) (size 0.8) (drill 0.4) (layers "F.Cu" "B.Cu") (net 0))
 (via (at 53.759488 119.665808) (size 0.8) (drill 0.4) (layers "F.Cu" "B.Cu") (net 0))
 (via (at 77.185212 122.124942) (size 0.8) (drill 0.4) (layers "F.Cu" "B.Cu") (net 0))
 (via (at 57.439431 123.231966) (size 0.8) (drill 0.4) (layers "F.Cu" "B.Cu") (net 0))
 (via (at 78.363713 115.39358) (size 0.8) (drill 0.4) (layers "F.Cu" "B.Cu") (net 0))
 (segment (start 81.368299 121.635848) (end 79.842274 119.456465) (width 0.25) (layer "B.Cu") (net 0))
 (segment (start 84.509835 122.189786) (end 83.632912 127.163066) (width 0.25) (layer "B.Cu") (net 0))
 (segment (start 70.438162 129.418619) (end 70.463165 129.443618) (width 0.25) (layer "B.Cu") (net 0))
 (segment (start 78.947537 119.362842) (end 79.669572 119.426013) (width 0.25) (layer "B.Cu") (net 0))
 (segment (start 86.14137 116.593709) (end 87.569339 116.845495) (width 0.25) (layer "B.Cu") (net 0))
 (segment (start 55.140407 119.918049) (end 55.555381 119.423497) (width 0.25) (layer "B.Cu") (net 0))
 (segment (start 49.002201 120.108762) (end 51.269063 119.709056) (width 0.25) (layer "B.Cu") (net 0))
 (segment (start 70.463171 129.443619) (end 67.273169 129.443617) (width 0.25) (layer "B.Cu") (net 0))
 (segment (start 113.592557 123.947463) (end 113.592557 126.60951) (width 0.2) (layer "B.Cu") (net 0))
 (segment (start 54.65125 122.074741) (end 55.816207 121.972822) (width 0.25) (layer "B.Cu") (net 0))
 (segment (start 78.363713 115.39358) (end 76.644067 116.836533) (width 0.25) (layer "B.Cu") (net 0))
 (segment (start 107.593228 121.82047) (end 108.955784 122.316407) (width 0.25) (layer "B.Cu") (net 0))
 (segment (start 70.438163 115.219247) (end 68.988167 115.21925) (width 0.25) (layer "B.Cu") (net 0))
 (segment (start 111.882792 126.788392) (end 108.824675 125.675331) (width 0.25) (layer "B.Cu") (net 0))
 (segment (start 56.276047 121.424805) (end 56.206328 120.627848) (width 0.25) (layer "B.Cu") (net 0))
 (segment (start 55.816207 121.972822) (end 56.276047 121.424805) (width 0.25) (layer "B.Cu") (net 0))
 (segment (start 92.394903 117.69637) (end 90.614614 127.792879) (width 0.25) (layer "B.Cu") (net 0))
 (segment (start 78.389735 119.8309) (end 78.947537 119.362842) (width 0.25) (layer "B.Cu") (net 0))
 (segment (start 63.453164 126.063621) (end 62.263172 127.253618) (width 0.25) (layer "B.Cu") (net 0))
 (segment (start 50.302396 127.482509) (end 50.197649 126.888463) (width 0.25) (layer "B.Cu") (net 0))
 (segment (start 84.509835 122.189786) (end 81.368295 121.63585) (width 0.25) (layer "B.Cu") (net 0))
 (segment (start 43.386178 128.483712) (end 42.420898 129.862275) (width 0.25) (layer "B.Cu") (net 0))
 (segment (start 79.316205 120.715009) (end 78.922846 125.211101) (width 0.25) (layer "B.Cu") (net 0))
 (segment (start 92.3949 117.696374) (end 90.966925 117.444586) (width 0.25) (layer "B.Cu") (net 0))
 (segment (start 112.244987 127.679112) (end 111.850528 126.833186) (width 0.25) (layer "B.Cu") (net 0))
 (segment (start 107.354031 122.521513) (end 107.625511 121.775637) (width 0.25) (layer "B.Cu") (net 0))
 (segment (start 48.381955 116.591152) (end 50.197649 126.888463) (width 0.25) (layer "B.Cu") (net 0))
 (segment (start 67.273169 129.443617) (end 67.26317 129.453619) (width 0.25) (layer "B.Cu") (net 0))
 (segment (start 59.463789 120.342855) (end 60.263171 121.013621) (width 0.25) (layer "B.Cu") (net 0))
 (segment (start 50.876608 130.595089) (end 47.735073 131.149026) (width 0.25) (layer "B.Cu") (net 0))
 (segment (start 59.063174 127.253619) (end 62.263172 127.253618) (width 0.25) (layer "B.Cu") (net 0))
 (segment (start 112.197725 123.49637) (end 113.560279 123.992296) (width 0.25) (layer "B.Cu") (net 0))
 (segment (start 89.929204 131.680027) (end 89.949482 131.708987) (width 0.25) (layer "B.Cu") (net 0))
 (segment (start 90.474462 128.587723) (end 90.614614 127.792879) (width 0.25) (layer "B.Cu") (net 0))
 (segment (start 108.824675 125.675331) (end 107.354031 122.521513) (width 0.25) (layer "B.Cu") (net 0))
 (segment (start 105.708327 136.282277) (end 108.705948 137.373318) (width 0.25) (layer "B.Cu") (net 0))
 (segment (start 53.916294 121.458037) (end 54.65125 122.074741) (width 0.25) (layer "B.Cu") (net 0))
 (segment (start 78.320012 120.627855) (end 78.389735 119.8309) (width 0.25) (layer "B.Cu") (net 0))
 (segment (start 70.438165 115.219251) (end 70.438165 124.820533) (width 0.25) (layer "B.Cu") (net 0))
 (segment (start 78.922846 125.211101) (end 76.534015 127.215565) (width 0.25) (layer "B.Cu") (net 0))
 (segment (start 89.94948 131.708984) (end 86.807944 131.155046) (width 0.25) (layer "B.Cu") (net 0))
 (segment (start 110.208388 133.274628) (end 112.244987 127.679112) (width 0.25) (layer "B.Cu") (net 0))
 (segment (start 53.759488 119.665808) (end 53.916294 121.458037) (width 0.25) (layer "B.Cu") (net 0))
 (segment (start 64.054536 115.219247) (end 64.088168 115.219248) (width 0.25) (layer "B.Cu") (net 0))
 (segment (start 113.592557 123.947463) (end 113.592557 125.078627) (width 0.2) (layer "B.Cu") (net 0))
 (segment (start 70.438166 118.791123) (end 72.739992 118.791121) (width 0.25) (layer "B.Cu") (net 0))
 (segment (start 57.437858 123.230646) (end 57.202519 120.540696) (width 0.25) (layer "B.Cu") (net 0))
 (segment (start 113.592557 125.078627) (end 111.882793 126.788391) (width 0.2) (layer "B.Cu") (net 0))
 (segment (start 101.762312 132.504852) (end 103.287543 131.793624) (width 0.25) (layer "B.Cu") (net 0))
 (segment (start 91.808019 121.242477) (end 94.074872 121.642189) (width 0.25) (layer "B.Cu") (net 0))
 (segment (start 98.755292 131.410385) (end 101.762312 132.504852) (width 0.25) (layer "B.Cu") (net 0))
 (segment (start 64.088166 115.21925) (end 65.538165 115.219247) (width 0.25) (layer "B.Cu") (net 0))
 (segment (start 39.269515 130.417951) (end 42.420898 129.862275) (width 0.25) (layer "B.Cu") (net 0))
 (segment (start 42.128424 117.693815) (end 43.556396 117.442027) (width 0.25) (layer "B.Cu") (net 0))
 (segment (start 76.644067 116.836533) (end 76.327622 120.453537) (width 0.25) (layer "B.Cu") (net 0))
 (segment (start 50.847651 130.574809) (end 50.876611 130.595086) (width 0.25) (layer "B.Cu") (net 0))
 (segment (start 86.796361 131.163158) (end 90.474462 128.587723) (width 0.25) (layer "B.Cu") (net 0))
 (segment (start 70.438164 126.278626) (end 70.438165 124.820533) (width 0.25) (layer "B.Cu") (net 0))
 (segment (start 55.210131 120.715008) (end 55.140407 119.918049) (width 0.25) (layer "B.Cu") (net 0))
 (segment (start 47.735073 131.149026) (end 47.72696 131.160611) (width 0.25) (layer "B.Cu") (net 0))
 (segment (start 47.726959 131.160613) (end 50.302396 127.482509) (width 0.25) (layer "B.Cu") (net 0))
 (segment (start 83.632912 127.163066) (end 82.254347 128.128342) (width 0.25) (layer "B.Cu") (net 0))
 (segment (start 79.842274 119.456465) (end 79.669572 119.426013) (width 0.25) (layer "B.Cu") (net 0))
 (segment (start 39.367722 124.064368) (end 42.509256 123.510434) (width 0.25) (layer "B.Cu") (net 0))
 (segment (start 108.705948 137.373318) (end 108.718763 137.367347) (width 0.25) (layer "B.Cu") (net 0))
 (segment (start 57.439431 123.231966) (end 57.437858 123.230646) (width 0.25) (layer "B.Cu") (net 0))
 (segment (start 109.822846 134.333898) (end 110.208388 133.274628) (width 0.25) (layer "B.Cu") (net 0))
 (segment (start 78.922846 125.211101) (end 78.445627 125.611534) (width 0.25) (layer "B.Cu") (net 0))
 (segment (start 111.972762 127.095319) (end 114.135767 127.882592) (width 0.25) (layer "B.Cu") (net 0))
 (segment (start 58.198715 120.453537) (end 59.463789 120.342855) (width 0.25) (layer "B.Cu") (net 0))
 (segment (start 113.592557 126.60951) (end 114.852221 127.869174) (width 0.2) (layer "B.Cu") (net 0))
 (segment (start 102.017128 125.957132) (end 105.014743 127.048175) (width 0.25) (layer "B.Cu") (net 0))
 (segment (start 60.26207 119.011717) (end 64.054536 115.219247) (width 0.25) (layer "B.Cu") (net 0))
 (segment (start 42.509256 123.510434) (end 43.386178 128.483712) (width 0.25) (layer "B.Cu") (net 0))
 (segment (start 46.953983 116.842941) (end 48.381955 116.591151) (width 0.25) (layer "B.Cu") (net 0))
 (segment (start 67.263171 129.453617) (end 70.438164 126.278626) (width 0.25) (layer "B.Cu") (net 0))
 (segment (start 86.807944 131.155046) (end 86.796359 131.163158) (width 0.25) (layer "B.Cu") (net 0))
 (segment (start 55.555381 119.423497) (end 60.26207 119.011717) (width 0.25) (layer "B.Cu") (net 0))
 (segment (start 103.287543 131.793624) (end 105.014743 127.048175) (width 0.25) (layer "B.Cu") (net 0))
 (segment (start 63.453169 121.013619) (end 63.453164 126.063621) (width 0.25) (layer "B.Cu") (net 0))
 (segment (start 77.185212 122.124942) (end 77.323814 120.540692) (width 0.25) (layer "B.Cu") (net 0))
 (segment (start 60.263168 121.013618) (end 63.453169 121.013619) (width 0.25) (layer "B.Cu") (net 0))
 (segment (start 82.254347 128.128342) (end 79.102959 127.572669) (width 0.25) (layer "B.Cu") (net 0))
 (segment (start 105.740592 136.237485) (end 109.822846 134.333898) (width 0.25) (layer "B.Cu") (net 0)))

